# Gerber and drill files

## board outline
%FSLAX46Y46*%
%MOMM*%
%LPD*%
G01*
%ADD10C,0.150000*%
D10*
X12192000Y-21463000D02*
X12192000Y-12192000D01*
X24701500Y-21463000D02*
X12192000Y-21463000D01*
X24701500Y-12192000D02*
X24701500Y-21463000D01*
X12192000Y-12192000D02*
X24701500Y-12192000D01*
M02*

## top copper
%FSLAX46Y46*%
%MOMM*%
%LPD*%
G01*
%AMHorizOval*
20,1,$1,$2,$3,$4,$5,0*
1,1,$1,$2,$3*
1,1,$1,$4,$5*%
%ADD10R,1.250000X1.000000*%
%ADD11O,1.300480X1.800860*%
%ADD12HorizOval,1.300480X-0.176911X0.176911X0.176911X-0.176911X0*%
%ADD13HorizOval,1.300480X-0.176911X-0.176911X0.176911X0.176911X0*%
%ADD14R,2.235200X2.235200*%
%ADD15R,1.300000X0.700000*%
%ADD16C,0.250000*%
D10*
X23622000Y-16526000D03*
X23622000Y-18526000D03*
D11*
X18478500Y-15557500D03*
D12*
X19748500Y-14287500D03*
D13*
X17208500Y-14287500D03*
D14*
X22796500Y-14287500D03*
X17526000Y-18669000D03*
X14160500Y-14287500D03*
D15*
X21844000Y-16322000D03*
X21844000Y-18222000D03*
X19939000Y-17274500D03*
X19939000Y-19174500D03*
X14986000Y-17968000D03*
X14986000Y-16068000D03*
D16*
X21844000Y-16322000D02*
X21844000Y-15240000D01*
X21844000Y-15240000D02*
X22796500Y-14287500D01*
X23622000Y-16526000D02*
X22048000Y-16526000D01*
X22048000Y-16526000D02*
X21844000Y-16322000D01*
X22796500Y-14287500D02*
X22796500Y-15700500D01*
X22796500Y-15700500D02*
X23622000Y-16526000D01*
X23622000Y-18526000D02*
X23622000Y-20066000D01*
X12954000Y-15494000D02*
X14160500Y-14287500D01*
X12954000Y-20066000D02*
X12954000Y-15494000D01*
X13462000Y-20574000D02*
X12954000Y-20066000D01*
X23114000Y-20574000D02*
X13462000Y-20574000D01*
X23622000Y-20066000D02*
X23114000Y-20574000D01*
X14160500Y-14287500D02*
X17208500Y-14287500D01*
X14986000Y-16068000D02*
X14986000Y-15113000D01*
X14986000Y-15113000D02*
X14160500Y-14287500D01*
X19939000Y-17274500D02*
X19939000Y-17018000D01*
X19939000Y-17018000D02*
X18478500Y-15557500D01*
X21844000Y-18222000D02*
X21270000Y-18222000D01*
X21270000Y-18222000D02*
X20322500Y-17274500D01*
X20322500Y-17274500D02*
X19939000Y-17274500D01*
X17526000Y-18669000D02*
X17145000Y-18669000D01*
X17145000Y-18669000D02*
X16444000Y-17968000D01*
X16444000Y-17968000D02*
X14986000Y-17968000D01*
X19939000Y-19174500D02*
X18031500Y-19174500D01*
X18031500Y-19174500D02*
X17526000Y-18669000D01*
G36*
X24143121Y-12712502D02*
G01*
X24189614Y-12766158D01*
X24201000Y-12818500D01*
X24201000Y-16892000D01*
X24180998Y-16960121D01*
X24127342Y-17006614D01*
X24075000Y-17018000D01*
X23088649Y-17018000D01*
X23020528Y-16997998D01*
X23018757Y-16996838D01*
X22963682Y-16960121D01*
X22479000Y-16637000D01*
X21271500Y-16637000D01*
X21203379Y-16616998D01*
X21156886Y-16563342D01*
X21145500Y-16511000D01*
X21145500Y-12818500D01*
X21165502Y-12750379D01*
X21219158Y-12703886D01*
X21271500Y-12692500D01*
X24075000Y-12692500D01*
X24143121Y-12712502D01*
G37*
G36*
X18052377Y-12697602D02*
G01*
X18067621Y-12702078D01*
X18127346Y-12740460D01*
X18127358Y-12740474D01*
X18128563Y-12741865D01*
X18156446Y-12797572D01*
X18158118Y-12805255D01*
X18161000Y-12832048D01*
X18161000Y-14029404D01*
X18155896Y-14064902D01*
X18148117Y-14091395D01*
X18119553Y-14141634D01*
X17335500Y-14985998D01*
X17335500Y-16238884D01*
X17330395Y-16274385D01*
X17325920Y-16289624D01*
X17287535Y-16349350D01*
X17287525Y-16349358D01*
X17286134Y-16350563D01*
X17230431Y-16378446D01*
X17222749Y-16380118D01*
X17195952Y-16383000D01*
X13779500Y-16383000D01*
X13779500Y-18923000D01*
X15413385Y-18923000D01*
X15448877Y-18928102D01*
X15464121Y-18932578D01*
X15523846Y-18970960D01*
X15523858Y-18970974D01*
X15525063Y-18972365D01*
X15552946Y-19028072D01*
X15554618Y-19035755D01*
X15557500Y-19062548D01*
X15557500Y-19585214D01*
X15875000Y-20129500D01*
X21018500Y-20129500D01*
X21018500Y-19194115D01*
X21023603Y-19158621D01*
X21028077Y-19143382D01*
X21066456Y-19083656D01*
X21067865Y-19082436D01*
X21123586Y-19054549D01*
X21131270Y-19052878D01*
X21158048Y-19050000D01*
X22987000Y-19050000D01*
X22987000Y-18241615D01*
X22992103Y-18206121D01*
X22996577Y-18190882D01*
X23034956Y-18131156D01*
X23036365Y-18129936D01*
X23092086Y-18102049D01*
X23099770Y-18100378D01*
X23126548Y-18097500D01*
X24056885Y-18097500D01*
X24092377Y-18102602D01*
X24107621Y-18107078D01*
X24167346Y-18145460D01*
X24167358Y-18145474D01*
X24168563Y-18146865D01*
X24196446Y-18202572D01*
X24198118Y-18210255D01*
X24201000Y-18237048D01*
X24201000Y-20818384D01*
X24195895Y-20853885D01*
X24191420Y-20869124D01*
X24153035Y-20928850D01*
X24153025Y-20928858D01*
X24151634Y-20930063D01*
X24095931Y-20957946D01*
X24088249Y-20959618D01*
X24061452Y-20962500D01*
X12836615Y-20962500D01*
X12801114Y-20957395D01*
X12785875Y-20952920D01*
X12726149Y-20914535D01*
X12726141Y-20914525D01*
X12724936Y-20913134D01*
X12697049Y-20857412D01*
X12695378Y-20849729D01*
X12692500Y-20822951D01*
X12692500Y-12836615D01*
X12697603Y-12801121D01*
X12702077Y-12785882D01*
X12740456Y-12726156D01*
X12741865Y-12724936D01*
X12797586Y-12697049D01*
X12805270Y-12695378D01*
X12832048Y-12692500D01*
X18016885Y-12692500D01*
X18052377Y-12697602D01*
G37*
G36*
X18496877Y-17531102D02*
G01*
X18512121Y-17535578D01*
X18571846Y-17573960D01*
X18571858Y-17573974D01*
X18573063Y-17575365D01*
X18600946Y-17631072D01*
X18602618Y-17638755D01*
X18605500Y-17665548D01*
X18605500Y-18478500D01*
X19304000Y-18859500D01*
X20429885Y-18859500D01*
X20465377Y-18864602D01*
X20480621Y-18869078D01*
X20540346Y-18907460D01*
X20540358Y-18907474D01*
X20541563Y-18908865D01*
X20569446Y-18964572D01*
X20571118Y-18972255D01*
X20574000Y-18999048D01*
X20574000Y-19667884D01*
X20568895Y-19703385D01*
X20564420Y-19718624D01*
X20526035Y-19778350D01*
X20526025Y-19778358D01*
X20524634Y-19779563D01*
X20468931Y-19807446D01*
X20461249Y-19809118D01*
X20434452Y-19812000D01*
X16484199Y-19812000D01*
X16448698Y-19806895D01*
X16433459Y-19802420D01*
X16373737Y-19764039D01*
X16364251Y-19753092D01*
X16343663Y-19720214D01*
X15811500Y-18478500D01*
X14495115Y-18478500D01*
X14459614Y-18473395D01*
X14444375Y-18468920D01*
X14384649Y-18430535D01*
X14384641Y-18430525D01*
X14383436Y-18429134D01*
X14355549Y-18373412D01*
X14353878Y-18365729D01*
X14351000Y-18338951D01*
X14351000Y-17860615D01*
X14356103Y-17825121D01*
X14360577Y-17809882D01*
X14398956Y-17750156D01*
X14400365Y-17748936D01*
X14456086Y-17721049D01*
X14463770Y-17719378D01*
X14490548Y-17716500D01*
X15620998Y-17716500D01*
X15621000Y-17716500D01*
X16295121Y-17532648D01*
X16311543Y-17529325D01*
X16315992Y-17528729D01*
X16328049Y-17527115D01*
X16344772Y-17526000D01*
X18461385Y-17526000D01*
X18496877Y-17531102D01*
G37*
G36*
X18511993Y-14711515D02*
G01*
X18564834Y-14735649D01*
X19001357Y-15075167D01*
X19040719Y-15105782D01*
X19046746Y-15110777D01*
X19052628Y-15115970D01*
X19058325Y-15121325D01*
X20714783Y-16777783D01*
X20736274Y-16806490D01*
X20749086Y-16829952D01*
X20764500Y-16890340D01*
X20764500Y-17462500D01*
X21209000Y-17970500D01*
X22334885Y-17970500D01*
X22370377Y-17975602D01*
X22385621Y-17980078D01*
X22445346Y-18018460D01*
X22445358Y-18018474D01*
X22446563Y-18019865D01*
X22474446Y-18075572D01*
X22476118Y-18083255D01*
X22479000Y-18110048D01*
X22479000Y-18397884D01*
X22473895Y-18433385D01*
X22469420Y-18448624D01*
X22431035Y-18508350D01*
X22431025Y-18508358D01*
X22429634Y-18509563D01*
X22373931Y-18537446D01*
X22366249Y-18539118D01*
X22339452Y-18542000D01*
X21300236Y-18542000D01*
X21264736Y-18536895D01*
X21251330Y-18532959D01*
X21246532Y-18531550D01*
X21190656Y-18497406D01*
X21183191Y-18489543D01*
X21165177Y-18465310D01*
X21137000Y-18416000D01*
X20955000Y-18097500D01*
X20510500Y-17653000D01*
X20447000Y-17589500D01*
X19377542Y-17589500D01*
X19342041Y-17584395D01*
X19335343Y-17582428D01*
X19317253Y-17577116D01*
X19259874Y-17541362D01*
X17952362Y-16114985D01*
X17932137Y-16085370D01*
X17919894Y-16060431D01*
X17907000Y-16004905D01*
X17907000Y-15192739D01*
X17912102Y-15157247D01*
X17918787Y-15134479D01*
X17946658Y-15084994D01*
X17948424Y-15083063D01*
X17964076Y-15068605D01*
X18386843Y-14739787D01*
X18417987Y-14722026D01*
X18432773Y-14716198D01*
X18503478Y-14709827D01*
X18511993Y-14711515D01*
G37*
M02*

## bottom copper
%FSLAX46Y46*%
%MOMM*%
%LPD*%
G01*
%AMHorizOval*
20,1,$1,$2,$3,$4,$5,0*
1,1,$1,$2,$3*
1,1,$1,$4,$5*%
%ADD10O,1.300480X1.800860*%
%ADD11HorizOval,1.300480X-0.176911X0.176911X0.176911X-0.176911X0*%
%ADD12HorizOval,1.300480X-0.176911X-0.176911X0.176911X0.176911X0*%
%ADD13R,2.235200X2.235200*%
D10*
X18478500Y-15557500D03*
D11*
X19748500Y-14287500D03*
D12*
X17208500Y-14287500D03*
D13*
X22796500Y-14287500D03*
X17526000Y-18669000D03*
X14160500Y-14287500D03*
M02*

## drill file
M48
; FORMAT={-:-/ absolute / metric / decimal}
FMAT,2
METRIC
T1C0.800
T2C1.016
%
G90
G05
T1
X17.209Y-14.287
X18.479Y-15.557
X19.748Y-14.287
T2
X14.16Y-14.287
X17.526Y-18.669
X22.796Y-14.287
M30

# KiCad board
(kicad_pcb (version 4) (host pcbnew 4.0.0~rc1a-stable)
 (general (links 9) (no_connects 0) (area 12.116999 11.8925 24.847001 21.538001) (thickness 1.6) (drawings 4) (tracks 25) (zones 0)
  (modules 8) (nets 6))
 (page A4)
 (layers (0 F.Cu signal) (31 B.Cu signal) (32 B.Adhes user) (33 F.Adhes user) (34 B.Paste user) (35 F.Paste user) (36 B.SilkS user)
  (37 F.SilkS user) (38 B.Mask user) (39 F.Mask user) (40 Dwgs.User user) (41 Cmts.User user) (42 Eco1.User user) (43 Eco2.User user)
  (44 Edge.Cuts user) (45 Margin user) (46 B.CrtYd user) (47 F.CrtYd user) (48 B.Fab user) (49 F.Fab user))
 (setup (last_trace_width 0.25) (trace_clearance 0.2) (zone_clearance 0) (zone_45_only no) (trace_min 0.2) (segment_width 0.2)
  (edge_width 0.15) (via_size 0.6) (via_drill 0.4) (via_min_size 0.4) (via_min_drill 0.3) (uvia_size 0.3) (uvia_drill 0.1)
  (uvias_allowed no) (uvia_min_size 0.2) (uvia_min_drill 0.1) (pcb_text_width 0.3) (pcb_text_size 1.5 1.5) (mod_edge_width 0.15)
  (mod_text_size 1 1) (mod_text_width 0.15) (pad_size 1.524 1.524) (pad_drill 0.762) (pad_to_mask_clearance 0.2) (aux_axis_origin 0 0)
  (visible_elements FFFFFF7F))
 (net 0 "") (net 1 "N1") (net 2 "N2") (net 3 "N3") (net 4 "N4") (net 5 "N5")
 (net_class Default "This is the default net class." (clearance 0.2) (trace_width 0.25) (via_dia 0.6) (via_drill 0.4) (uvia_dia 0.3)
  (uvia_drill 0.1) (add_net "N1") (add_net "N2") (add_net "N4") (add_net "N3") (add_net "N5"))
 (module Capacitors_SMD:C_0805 (layer F.Cu) (at 23.622 17.526 270)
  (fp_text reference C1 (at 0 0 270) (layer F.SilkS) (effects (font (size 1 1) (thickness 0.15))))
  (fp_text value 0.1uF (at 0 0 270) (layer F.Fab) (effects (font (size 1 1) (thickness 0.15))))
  (pad 1 smd rect (at -1 0 270) (size 1 1.25) (layers F.Cu F.Paste F.Mask) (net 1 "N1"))
  (pad 2 smd rect (at 1 0 270) (size 1 1.25) (layers F.Cu F.Paste F.Mask) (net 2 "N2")))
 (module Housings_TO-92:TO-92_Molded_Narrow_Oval (layer F.Cu) (at 19.7485 14.2875 180)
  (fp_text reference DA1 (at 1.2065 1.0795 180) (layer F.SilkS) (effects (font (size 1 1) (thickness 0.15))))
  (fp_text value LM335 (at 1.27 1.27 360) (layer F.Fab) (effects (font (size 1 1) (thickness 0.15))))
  (pad 2 thru_hole oval (at 1.27 -1.27 270) (size 1.80086 1.30048) (drill 0.8) (layers *.Cu *.Mask F.SilkS) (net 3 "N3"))
  (pad 1 thru_hole oval (at 0 0 225) (size 1.30048 1.80086) (drill 0.8) (layers *.Cu *.Mask F.SilkS) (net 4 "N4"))
  (pad 3 thru_hole oval (at 2.54 0 225) (size 1.80086 1.30048) (drill 0.8) (layers *.Cu *.Mask F.SilkS) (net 2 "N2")))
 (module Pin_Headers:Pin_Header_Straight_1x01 (layer F.Cu) (at 22.7965 14.2875)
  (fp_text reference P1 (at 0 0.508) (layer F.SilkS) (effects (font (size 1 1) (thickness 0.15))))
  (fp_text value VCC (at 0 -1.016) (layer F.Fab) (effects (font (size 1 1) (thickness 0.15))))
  (pad 1 thru_hole rect (at 0 0) (size 2.2352 2.2352) (drill 1.016) (layers *.Cu *.Mask F.SilkS) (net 1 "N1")))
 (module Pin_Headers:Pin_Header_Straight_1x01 (layer F.Cu) (at 17.526 18.669)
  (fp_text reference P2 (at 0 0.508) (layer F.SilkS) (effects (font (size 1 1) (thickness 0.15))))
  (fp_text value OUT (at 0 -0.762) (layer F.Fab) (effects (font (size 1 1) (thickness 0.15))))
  (pad 1 thru_hole rect (at 0 0) (size 2.2352 2.2352) (drill 1.016) (layers *.Cu *.Mask F.SilkS) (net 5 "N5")))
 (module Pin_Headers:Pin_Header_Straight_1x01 (layer F.Cu) (at 14.1605 14.2875)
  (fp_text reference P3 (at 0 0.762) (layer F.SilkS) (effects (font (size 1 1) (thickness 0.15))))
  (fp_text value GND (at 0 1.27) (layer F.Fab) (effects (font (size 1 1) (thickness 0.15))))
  (pad 1 thru_hole rect (at 0 0) (size 2.2352 2.2352) (drill 1.016) (layers *.Cu *.Mask F.SilkS) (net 2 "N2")))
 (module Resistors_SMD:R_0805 (layer F.Cu) (at 21.844 17.272 270)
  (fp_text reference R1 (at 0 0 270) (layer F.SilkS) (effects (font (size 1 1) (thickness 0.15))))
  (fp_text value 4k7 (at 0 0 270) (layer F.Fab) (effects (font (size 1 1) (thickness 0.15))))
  (pad 1 smd rect (at -0.95 0 270) (size 0.7 1.3) (layers F.Cu F.Paste F.Mask) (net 1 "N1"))
  (pad 2 smd rect (at 0.95 0 270) (size 0.7 1.3) (layers F.Cu F.Paste F.Mask) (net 3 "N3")))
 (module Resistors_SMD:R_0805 (layer F.Cu) (at 19.939 18.2245 270)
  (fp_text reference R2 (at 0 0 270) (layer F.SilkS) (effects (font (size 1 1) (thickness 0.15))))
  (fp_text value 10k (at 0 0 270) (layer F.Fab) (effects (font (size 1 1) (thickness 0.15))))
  (pad 1 smd rect (at -0.95 0 270) (size 0.7 1.3) (layers F.Cu F.Paste F.Mask) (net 3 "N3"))
  (pad 2 smd rect (at 0.95 0 270) (size 0.7 1.3) (layers F.Cu F.Paste F.Mask) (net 5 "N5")))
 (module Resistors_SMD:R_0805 (layer F.Cu) (at 14.986 17.018 90)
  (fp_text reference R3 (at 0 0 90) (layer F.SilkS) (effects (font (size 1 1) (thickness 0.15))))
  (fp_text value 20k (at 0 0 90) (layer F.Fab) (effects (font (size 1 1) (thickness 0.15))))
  (pad 1 smd rect (at -0.95 0 90) (size 0.7 1.3) (layers F.Cu F.Paste F.Mask) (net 5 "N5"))
  (pad 2 smd rect (at 0.95 0 90) (size 0.7 1.3) (layers F.Cu F.Paste F.Mask) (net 2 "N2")))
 (gr_line (start 12.192 21.463) (end 12.192 12.192) (angle 90) (layer Edge.Cuts) (width 0.15))
 (gr_line (start 24.7015 21.463) (end 12.192 21.463) (angle 90) (layer Edge.Cuts) (width 0.15))
 (gr_line (start 24.7015 12.192) (end 24.7015 21.463) (angle 90) (layer Edge.Cuts) (width 0.15))
 (gr_line (start 12.192 12.192) (end 24.7015 12.192) (angle 90) (layer Edge.Cuts) (width 0.15))
 (segment (start 21.844 16.322) (end 21.844 15.24) (width 0.25) (layer F.Cu) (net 1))
 (segment (start 21.844 15.24) (end 22.7965 14.2875) (width 0.25) (layer F.Cu) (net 1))
 (segment (start 23.622 16.526) (end 22.048 16.526) (width 0.25) (layer F.Cu) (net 1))
 (segment (start 22.048 16.526) (end 21.844 16.322) (width 0.25) (layer F.Cu) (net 1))
 (segment (start 22.7965 14.2875) (end 22.7965 15.7005) (width 0.25) (layer F.Cu) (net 1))
 (segment (start 22.7965 15.7005) (end 23.622 16.526) (width 0.25) (layer F.Cu) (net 1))
 (segment (start 23.622 18.526) (end 23.622 20.066) (width 0.25) (layer F.Cu) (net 2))
 (segment (start 12.954 15.494) (end 14.1605 14.2875) (width 0.25) (layer F.Cu) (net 2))
 (segment (start 12.954 20.066) (end 12.954 15.494) (width 0.25) (layer F.Cu) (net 2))
 (segment (start 13.462 20.574) (end 12.954 20.066) (width 0.25) (layer F.Cu) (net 2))
 (segment (start 23.114 20.574) (end 13.462 20.574) (width 0.25) (layer F.Cu) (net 2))
 (segment (start 23.622 20.066) (end 23.114 20.574) (width 0.25) (layer F.Cu) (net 2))
 (segment (start 14.1605 14.2875) (end 17.2085 14.2875) (width 0.25) (layer F.Cu) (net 2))
 (segment (start 14.986 16.068) (end 14.986 15.113) (width 0.25) (layer F.Cu) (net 2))
 (segment (start 14.986 15.113) (end 14.1605 14.2875) (width 0.25) (layer F.Cu) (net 2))
 (segment (start 19.939 17.2745) (end 19.939 17.018) (width 0.25) (layer F.Cu) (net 3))
 (segment (start 19.939 17.018) (end 18.4785 15.5575) (width 0.25) (layer F.Cu) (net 3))
 (segment (start 21.844 18.222) (end 21.27 18.222) (width 0.25) (layer F.Cu) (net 3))
 (segment (start 21.27 18.222) (end 20.3225 17.2745) (width 0.25) (layer F.Cu) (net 3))
 (segment (start 20.3225 17.2745) (end 19.939 17.2745) (width 0.25) (layer F.Cu) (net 3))
 (segment (start 17.526 18.669) (end 17.145 18.669) (width 0.25) (layer F.Cu) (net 5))
 (segment (start 17.145 18.669) (end 16.444 17.968) (width 0.25) (layer F.Cu) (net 5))
 (segment (start 16.444 17.968) (end 14.986 17.968) (width 0.25) (layer F.Cu) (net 5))
 (segment (start 19.939 19.1745) (end 18.0315 19.1745) (width 0.25) (layer F.Cu) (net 5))
 (segment (start 18.0315 19.1745) (end 17.526 18.669) (width 0.25) (layer F.Cu) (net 5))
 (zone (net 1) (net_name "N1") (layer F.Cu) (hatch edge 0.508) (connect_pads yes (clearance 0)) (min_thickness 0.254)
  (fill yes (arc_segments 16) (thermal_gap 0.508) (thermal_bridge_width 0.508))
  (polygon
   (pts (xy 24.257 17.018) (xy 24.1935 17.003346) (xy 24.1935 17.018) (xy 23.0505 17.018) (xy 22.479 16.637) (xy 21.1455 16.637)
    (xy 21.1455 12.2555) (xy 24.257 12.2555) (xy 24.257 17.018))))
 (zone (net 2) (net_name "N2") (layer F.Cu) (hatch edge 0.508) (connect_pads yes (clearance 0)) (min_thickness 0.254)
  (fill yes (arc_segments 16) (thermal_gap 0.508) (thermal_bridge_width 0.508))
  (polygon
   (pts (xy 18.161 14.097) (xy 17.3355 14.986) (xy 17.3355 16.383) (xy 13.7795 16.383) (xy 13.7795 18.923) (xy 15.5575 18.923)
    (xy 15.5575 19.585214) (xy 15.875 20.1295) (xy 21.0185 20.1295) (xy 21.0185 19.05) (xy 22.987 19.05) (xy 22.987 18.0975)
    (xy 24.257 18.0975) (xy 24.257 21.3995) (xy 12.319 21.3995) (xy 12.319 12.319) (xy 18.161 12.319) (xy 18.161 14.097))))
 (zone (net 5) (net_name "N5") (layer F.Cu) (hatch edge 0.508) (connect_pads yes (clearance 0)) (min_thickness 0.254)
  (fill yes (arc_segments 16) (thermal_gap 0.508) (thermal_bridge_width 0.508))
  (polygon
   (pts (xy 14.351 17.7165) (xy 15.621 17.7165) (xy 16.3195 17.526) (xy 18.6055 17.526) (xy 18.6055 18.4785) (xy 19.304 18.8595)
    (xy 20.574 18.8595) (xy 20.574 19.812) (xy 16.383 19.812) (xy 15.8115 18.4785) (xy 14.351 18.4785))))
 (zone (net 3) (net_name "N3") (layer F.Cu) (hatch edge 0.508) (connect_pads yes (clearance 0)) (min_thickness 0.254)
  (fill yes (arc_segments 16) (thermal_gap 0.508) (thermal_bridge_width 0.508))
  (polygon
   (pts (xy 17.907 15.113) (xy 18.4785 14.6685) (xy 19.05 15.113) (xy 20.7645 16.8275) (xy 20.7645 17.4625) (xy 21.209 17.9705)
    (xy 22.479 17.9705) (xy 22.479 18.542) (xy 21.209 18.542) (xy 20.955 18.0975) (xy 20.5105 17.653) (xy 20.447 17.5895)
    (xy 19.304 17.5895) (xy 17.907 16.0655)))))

